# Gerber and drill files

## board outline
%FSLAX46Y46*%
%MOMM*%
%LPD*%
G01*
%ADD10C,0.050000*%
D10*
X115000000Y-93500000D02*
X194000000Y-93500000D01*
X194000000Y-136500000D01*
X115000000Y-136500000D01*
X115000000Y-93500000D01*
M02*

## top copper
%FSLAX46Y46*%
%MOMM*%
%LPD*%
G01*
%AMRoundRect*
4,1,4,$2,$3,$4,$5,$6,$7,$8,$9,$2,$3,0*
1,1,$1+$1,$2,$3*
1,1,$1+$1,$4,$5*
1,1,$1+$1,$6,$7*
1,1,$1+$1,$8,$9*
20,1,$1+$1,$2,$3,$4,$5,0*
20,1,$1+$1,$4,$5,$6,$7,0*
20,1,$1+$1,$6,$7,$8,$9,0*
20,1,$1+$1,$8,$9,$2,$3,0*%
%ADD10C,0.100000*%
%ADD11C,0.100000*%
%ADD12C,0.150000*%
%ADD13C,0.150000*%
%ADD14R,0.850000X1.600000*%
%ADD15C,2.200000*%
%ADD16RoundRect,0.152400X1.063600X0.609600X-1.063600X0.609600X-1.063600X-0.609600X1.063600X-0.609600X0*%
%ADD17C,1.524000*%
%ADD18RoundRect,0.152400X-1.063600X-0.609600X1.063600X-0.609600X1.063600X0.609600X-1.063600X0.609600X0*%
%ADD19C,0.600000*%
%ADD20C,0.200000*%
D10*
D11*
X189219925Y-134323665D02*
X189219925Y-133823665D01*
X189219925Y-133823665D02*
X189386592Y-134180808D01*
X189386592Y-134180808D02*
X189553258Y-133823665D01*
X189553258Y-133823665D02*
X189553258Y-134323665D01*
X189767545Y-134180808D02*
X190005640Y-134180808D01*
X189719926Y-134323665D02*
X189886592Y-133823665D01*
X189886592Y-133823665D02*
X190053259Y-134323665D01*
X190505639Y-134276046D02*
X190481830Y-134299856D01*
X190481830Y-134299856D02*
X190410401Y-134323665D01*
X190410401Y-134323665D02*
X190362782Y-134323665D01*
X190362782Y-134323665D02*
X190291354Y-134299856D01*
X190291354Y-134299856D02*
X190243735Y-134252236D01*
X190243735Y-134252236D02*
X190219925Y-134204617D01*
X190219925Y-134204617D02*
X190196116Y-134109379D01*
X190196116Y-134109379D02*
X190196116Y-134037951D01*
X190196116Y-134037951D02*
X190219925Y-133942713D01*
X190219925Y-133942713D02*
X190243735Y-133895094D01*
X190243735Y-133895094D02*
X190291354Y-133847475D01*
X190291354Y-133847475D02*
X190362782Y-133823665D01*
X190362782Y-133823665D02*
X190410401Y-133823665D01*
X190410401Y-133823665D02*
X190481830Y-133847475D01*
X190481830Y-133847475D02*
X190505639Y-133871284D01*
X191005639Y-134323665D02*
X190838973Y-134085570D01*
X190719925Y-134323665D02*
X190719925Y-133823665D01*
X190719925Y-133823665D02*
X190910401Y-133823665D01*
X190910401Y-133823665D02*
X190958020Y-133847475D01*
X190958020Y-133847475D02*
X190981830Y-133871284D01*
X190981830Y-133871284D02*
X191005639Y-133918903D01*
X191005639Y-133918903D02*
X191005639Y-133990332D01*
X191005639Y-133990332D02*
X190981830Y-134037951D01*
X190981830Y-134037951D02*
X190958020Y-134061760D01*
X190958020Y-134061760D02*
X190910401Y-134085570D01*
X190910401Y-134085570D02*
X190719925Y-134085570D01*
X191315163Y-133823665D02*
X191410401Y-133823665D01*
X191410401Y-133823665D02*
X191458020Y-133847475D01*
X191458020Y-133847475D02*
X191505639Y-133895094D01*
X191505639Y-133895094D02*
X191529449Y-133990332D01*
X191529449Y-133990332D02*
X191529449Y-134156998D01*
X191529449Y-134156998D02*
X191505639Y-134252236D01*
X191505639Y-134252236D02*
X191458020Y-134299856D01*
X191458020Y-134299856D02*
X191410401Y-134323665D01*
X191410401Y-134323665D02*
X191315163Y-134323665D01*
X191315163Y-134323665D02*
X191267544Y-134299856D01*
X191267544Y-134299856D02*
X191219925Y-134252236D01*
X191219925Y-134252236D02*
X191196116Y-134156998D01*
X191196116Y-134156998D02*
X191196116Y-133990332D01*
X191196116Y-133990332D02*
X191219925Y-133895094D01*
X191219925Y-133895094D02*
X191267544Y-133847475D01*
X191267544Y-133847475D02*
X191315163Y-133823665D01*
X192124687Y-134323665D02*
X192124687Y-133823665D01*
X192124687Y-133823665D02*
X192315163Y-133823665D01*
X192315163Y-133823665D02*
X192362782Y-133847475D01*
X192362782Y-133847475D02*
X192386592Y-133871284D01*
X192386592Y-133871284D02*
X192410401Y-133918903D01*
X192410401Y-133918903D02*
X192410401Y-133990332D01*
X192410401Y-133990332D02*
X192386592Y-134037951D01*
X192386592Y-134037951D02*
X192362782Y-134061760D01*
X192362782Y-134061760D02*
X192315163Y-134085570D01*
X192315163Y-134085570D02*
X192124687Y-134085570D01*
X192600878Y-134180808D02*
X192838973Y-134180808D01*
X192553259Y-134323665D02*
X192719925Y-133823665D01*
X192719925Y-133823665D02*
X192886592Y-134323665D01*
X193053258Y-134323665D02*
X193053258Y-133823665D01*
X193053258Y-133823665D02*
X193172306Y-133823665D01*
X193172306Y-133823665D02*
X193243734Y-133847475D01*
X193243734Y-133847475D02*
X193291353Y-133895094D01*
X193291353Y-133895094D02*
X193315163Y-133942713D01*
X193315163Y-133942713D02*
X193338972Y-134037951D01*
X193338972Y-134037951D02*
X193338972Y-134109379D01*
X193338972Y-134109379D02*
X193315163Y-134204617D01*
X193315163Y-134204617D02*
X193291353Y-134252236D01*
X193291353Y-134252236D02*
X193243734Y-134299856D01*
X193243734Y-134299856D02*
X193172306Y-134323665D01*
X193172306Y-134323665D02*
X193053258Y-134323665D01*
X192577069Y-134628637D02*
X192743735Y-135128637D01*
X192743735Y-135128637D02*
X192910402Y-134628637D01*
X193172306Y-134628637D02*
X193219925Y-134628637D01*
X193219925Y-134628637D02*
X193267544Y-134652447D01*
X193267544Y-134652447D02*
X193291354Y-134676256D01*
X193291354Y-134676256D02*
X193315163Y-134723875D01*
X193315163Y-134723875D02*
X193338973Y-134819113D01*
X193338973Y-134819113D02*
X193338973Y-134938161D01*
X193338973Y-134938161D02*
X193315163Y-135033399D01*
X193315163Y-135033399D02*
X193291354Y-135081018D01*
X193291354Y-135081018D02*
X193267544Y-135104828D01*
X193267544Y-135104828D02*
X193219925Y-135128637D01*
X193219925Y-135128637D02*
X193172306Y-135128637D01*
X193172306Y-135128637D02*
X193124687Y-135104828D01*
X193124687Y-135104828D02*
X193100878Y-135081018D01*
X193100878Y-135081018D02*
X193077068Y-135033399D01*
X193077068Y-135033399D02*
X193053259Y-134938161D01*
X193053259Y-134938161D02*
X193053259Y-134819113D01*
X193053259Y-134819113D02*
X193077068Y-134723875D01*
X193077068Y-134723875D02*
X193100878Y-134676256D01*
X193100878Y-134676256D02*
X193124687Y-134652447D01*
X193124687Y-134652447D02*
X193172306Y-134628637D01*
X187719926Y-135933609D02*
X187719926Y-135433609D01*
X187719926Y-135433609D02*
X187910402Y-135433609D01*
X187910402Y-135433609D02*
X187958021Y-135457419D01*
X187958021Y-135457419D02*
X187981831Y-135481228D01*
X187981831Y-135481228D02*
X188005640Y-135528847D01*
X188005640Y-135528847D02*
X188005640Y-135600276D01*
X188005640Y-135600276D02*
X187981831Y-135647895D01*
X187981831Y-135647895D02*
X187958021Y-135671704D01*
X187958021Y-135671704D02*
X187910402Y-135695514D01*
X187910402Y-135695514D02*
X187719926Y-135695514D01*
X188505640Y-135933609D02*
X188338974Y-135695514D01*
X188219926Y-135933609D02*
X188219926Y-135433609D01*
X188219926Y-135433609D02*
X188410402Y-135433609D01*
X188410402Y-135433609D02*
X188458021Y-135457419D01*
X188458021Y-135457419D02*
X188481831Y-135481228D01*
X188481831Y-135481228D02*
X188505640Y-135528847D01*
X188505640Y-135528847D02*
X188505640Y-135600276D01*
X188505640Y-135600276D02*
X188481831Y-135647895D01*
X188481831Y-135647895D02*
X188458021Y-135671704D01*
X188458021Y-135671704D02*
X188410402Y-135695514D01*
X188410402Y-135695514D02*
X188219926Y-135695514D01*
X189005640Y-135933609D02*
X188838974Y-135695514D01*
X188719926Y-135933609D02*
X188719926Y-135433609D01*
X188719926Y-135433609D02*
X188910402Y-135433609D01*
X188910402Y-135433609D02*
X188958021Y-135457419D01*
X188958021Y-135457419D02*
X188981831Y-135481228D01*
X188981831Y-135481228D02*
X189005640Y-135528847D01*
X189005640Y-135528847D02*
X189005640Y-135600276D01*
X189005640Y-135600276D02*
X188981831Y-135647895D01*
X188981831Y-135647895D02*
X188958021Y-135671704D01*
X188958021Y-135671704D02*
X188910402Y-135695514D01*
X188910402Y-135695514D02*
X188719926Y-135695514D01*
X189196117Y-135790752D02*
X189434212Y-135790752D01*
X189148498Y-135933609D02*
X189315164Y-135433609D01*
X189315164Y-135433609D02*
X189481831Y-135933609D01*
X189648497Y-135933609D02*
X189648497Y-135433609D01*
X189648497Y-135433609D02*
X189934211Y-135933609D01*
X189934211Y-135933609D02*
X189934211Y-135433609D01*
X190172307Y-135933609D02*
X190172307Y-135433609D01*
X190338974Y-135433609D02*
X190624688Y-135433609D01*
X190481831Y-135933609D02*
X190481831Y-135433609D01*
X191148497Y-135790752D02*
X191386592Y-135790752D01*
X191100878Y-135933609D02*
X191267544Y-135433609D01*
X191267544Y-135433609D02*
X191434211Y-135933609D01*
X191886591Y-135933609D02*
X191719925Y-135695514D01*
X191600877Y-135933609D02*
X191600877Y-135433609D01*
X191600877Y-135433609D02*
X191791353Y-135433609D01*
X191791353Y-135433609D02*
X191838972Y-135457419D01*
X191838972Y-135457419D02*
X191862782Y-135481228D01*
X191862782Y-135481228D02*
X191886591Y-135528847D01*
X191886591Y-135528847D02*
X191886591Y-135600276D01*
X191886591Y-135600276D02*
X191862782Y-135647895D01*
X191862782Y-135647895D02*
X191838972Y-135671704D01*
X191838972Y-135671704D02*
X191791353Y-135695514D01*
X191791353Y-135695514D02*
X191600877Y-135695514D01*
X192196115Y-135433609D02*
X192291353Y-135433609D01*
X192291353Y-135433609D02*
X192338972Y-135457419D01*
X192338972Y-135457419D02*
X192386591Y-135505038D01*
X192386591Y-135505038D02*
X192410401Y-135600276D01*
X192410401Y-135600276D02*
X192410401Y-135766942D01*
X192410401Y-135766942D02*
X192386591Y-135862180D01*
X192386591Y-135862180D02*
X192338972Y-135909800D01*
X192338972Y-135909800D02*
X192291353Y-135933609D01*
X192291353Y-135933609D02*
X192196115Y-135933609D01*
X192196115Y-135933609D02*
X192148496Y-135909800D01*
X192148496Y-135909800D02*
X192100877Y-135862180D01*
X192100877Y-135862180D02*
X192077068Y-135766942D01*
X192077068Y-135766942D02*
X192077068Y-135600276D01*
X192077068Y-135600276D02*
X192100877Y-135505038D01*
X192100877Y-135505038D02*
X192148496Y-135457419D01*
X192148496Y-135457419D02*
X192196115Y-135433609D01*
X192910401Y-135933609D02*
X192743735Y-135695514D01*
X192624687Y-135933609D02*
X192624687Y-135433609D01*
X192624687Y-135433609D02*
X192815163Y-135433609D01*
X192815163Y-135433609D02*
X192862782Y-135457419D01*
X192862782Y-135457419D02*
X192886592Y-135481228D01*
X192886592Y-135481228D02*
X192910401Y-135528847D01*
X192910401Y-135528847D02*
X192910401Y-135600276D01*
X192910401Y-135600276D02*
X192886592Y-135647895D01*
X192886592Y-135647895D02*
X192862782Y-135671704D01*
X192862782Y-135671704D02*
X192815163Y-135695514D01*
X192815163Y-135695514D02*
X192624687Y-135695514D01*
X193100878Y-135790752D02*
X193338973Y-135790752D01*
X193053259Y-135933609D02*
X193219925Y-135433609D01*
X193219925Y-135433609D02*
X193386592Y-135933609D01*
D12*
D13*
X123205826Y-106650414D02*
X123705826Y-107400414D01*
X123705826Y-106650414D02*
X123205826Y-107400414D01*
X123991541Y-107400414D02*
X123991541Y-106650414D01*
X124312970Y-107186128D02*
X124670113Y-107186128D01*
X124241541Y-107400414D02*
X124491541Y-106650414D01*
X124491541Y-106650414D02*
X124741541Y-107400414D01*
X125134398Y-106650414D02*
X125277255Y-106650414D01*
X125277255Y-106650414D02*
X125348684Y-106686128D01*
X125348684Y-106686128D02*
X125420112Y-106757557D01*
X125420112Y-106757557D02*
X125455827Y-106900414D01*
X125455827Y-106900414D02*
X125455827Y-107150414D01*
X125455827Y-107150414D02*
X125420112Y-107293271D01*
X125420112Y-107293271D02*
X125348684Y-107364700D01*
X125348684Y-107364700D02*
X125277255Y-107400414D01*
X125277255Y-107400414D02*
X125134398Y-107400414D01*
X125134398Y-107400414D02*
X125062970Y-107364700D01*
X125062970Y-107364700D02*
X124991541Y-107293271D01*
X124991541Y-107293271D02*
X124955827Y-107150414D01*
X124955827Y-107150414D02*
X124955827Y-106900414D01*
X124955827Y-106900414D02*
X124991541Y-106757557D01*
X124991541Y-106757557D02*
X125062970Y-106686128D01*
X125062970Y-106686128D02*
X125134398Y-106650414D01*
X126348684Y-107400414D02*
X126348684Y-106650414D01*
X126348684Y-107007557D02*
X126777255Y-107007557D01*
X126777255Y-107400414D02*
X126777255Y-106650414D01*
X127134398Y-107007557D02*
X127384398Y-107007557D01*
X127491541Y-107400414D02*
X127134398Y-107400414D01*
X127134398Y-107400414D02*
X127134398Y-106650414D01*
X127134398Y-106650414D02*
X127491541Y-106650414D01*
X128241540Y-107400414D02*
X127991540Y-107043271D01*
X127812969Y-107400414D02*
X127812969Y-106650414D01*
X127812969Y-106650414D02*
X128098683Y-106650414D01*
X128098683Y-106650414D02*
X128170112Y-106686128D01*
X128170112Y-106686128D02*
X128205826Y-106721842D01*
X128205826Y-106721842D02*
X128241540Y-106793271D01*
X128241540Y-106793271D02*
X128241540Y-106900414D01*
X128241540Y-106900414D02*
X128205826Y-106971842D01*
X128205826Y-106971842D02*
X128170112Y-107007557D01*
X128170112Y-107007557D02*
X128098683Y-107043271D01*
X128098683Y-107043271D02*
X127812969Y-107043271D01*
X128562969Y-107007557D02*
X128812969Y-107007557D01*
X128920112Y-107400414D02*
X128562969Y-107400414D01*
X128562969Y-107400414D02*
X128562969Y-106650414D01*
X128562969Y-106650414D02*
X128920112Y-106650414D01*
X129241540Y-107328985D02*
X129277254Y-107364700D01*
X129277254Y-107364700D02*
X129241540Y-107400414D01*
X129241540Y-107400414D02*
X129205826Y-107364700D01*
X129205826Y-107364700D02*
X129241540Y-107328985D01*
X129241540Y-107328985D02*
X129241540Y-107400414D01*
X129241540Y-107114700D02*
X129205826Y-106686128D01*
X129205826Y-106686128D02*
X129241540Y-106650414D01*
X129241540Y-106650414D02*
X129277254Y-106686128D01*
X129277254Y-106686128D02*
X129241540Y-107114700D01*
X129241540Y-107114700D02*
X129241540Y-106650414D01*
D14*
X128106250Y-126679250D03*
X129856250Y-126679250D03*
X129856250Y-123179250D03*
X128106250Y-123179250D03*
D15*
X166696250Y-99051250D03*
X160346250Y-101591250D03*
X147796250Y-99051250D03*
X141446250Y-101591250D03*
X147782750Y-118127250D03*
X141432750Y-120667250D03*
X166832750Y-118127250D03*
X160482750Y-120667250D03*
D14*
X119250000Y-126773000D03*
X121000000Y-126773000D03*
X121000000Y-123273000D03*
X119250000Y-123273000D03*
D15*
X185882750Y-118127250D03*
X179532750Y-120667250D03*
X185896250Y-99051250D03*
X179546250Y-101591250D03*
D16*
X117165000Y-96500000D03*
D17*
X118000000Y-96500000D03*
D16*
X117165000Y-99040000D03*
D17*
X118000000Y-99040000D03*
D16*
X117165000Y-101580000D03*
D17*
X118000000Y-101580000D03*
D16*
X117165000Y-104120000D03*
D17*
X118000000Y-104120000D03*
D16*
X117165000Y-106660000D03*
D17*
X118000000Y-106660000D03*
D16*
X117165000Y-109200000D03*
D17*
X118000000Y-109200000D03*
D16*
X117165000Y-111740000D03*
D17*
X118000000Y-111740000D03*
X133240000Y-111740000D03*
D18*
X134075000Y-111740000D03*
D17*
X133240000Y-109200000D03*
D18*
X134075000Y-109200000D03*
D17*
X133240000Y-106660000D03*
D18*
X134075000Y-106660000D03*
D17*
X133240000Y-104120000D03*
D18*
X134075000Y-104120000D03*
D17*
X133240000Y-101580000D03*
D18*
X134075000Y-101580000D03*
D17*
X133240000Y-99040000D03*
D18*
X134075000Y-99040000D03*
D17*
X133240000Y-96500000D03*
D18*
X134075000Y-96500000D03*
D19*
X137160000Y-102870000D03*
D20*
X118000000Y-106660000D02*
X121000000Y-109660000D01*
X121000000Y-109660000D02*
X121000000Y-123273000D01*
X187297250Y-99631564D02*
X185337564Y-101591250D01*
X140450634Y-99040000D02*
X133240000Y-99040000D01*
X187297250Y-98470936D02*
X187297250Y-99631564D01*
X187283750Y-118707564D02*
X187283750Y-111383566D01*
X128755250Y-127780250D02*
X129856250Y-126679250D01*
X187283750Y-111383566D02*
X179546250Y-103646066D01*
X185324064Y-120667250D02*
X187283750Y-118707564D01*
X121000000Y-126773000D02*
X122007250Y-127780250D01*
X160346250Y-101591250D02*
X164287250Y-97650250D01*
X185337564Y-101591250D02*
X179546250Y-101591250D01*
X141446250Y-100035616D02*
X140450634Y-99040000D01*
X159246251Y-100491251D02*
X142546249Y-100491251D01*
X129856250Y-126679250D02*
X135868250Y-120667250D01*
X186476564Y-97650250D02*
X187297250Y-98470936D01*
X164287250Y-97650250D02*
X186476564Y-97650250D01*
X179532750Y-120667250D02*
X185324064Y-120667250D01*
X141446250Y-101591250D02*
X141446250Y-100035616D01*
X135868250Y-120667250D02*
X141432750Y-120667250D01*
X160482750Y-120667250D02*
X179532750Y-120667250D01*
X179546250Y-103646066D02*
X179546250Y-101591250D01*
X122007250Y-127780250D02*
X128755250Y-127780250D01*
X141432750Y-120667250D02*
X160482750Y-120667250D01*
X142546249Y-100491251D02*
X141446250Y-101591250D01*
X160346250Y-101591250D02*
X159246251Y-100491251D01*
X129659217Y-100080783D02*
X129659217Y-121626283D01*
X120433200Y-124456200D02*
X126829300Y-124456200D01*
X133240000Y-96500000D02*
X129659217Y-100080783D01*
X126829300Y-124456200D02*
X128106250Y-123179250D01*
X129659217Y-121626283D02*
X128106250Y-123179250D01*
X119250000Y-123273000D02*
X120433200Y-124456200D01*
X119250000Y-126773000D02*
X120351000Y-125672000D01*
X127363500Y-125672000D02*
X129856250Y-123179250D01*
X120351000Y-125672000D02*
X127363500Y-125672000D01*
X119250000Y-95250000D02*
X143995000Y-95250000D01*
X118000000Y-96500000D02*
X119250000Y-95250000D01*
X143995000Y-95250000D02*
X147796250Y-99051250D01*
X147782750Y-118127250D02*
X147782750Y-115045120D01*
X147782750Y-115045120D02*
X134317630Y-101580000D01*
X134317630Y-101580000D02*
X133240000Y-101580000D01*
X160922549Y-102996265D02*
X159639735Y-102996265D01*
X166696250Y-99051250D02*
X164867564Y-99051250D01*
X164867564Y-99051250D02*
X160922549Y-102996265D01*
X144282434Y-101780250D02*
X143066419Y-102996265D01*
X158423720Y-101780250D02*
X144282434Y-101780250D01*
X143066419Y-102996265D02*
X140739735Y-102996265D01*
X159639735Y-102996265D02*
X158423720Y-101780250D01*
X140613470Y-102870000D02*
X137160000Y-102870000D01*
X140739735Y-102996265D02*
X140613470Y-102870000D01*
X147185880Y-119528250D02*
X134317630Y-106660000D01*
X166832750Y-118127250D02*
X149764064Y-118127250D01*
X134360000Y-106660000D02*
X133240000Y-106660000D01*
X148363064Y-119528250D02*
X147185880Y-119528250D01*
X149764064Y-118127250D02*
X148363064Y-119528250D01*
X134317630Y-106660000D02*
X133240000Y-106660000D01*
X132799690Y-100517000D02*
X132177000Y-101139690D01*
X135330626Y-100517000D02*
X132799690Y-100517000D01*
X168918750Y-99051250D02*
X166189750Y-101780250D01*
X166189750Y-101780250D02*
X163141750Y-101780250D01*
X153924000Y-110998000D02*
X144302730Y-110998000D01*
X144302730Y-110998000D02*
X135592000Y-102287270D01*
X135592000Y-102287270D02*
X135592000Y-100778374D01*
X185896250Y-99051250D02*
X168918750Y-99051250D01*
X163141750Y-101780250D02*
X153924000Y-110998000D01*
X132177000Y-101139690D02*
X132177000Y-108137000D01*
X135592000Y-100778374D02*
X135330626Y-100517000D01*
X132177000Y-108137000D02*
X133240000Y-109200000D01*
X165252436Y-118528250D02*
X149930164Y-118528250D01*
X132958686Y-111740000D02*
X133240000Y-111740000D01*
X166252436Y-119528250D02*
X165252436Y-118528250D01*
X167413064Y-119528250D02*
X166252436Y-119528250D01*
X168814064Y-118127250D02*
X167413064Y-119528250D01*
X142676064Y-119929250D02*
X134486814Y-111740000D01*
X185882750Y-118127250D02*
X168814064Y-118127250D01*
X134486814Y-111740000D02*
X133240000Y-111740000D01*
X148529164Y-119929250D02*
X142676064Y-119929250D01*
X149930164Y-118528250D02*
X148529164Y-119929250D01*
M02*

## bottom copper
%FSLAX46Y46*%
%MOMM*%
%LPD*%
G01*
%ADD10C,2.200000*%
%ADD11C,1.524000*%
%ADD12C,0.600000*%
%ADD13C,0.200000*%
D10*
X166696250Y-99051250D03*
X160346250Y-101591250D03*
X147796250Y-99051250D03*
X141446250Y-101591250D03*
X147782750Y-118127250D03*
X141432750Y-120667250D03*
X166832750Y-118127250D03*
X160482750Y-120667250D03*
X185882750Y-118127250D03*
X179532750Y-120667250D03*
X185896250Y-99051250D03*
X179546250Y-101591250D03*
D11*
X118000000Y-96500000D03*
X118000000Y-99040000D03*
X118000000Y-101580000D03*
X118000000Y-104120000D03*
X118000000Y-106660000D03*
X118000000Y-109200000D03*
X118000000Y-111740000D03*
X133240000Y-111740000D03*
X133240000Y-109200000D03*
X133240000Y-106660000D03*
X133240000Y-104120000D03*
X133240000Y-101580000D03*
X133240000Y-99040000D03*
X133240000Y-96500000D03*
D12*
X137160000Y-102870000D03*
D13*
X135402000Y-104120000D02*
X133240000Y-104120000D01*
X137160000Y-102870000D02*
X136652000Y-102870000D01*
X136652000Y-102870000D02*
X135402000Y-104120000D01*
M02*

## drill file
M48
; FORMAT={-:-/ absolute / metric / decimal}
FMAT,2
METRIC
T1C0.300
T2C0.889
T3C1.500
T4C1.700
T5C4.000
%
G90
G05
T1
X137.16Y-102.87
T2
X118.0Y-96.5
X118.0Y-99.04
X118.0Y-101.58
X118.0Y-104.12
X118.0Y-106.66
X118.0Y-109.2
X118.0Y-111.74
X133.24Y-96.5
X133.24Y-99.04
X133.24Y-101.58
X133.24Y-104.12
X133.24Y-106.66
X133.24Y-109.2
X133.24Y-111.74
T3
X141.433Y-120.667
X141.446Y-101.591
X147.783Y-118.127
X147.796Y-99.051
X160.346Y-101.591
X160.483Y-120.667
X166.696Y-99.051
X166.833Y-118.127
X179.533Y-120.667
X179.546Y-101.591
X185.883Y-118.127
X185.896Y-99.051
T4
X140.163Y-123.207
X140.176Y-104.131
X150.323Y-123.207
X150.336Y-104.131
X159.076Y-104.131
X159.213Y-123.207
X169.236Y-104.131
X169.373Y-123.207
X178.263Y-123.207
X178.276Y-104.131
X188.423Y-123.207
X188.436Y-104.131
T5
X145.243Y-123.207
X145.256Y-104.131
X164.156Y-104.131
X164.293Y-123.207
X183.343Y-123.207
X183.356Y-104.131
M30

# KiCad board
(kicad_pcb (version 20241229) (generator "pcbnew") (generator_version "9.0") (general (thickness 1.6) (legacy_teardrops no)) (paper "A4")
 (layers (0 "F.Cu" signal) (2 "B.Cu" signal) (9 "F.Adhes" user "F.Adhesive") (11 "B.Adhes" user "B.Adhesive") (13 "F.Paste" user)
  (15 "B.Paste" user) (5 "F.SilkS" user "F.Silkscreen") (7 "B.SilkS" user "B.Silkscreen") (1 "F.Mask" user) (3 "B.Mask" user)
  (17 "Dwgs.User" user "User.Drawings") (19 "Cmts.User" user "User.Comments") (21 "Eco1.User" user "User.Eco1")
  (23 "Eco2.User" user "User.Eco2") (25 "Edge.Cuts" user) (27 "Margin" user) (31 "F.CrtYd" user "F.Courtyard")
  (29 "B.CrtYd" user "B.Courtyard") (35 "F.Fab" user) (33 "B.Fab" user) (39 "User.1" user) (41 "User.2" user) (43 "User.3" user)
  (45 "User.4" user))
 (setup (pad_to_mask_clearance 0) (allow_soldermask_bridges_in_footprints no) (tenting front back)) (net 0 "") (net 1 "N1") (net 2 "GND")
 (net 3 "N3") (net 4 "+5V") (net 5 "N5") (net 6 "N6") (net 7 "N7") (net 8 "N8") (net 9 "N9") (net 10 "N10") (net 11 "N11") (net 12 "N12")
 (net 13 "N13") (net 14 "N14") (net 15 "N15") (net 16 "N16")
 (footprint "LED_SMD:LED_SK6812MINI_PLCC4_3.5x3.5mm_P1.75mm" (layer "F.Cu") (at 128.98125 124.92925 90)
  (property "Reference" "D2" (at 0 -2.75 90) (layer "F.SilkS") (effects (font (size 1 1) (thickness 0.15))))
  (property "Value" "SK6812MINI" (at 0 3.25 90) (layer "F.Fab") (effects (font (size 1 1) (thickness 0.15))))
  (pad "1" smd rect (at -1.75 -0.875 90) (size 1.6 0.85) (layers "F.Cu" "F.Mask" "F.Paste") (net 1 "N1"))
  (pad "2" smd rect (at -1.75 0.875 90) (size 1.6 0.85) (layers "F.Cu" "F.Mask" "F.Paste") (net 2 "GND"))
  (pad "3" smd rect (at 1.75 0.875 90) (size 1.6 0.85) (layers "F.Cu" "F.Mask" "F.Paste") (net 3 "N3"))
  (pad "4" smd rect (at 1.75 -0.875 90) (size 1.6 0.85) (layers "F.Cu" "F.Mask" "F.Paste") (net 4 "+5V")))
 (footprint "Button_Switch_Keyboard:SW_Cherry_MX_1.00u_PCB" (layer "F.Cu") (at 166.69625 99.05125)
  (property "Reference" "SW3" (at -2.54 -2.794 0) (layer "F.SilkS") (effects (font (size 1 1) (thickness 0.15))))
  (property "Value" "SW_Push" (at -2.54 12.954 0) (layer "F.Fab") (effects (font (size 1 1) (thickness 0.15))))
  (pad "" np_thru_hole circle (at -7.62 5.08) (size 1.7 1.7) (drill 1.7) (layers "*.Cu" "*.Mask"))
  (pad "" np_thru_hole circle (at -2.54 5.08) (size 4 4) (drill 4) (layers "*.Cu" "*.Mask"))
  (pad "" np_thru_hole circle (at 2.54 5.08) (size 1.7 1.7) (drill 1.7) (layers "*.Cu" "*.Mask"))
  (pad "1" thru_hole circle (at 0 0) (size 2.2 2.2) (drill 1.5) (layers "*.Cu" "*.Mask") (remove_unused_layers no) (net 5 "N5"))
  (pad "2" thru_hole circle (at -6.35 2.54) (size 2.2 2.2) (drill 1.5) (layers "*.Cu" "*.Mask") (remove_unused_layers no) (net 2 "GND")))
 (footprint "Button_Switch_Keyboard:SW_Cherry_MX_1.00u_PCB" (layer "F.Cu") (at 147.79625 99.05125)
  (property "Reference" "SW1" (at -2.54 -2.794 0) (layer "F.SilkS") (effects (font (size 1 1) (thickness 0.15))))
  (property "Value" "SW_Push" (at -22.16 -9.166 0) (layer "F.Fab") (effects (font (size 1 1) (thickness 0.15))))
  (pad "" np_thru_hole circle (at -7.62 5.08) (size 1.7 1.7) (drill 1.7) (layers "*.Cu" "*.Mask"))
  (pad "" np_thru_hole circle (at -2.54 5.08) (size 4 4) (drill 4) (layers "*.Cu" "*.Mask"))
  (pad "" np_thru_hole circle (at 2.54 5.08) (size 1.7 1.7) (drill 1.7) (layers "*.Cu" "*.Mask"))
  (pad "1" thru_hole circle (at 0 0) (size 2.2 2.2) (drill 1.5) (layers "*.Cu" "*.Mask") (remove_unused_layers no) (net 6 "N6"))
  (pad "2" thru_hole circle (at -6.35 2.54) (size 2.2 2.2) (drill 1.5) (layers "*.Cu" "*.Mask") (remove_unused_layers no) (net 2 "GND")))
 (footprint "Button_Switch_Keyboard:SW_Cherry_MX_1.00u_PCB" (layer "F.Cu") (at 147.78275 118.12725)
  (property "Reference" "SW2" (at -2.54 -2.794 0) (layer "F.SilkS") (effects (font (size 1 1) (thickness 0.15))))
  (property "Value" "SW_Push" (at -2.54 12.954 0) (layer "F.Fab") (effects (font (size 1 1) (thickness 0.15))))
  (pad "" np_thru_hole circle (at -7.62 5.08) (size 1.7 1.7) (drill 1.7) (layers "*.Cu" "*.Mask"))
  (pad "" np_thru_hole circle (at -2.54 5.08) (size 4 4) (drill 4) (layers "*.Cu" "*.Mask"))
  (pad "" np_thru_hole circle (at 2.54 5.08) (size 1.7 1.7) (drill 1.7) (layers "*.Cu" "*.Mask"))
  (pad "1" thru_hole circle (at 0 0) (size 2.2 2.2) (drill 1.5) (layers "*.Cu" "*.Mask") (remove_unused_layers no) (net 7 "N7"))
  (pad "2" thru_hole circle (at -6.35 2.54) (size 2.2 2.2) (drill 1.5) (layers "*.Cu" "*.Mask") (remove_unused_layers no) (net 2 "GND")))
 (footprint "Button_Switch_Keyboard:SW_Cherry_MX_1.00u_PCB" (layer "F.Cu") (at 166.83275 118.12725)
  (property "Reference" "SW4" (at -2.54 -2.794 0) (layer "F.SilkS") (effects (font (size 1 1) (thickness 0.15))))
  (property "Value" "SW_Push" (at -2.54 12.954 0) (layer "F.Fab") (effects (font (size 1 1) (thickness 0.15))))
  (pad "" np_thru_hole circle (at -7.62 5.08) (size 1.7 1.7) (drill 1.7) (layers "*.Cu" "*.Mask"))
  (pad "" np_thru_hole circle (at -2.54 5.08) (size 4 4) (drill 4) (layers "*.Cu" "*.Mask"))
  (pad "" np_thru_hole circle (at 2.54 5.08) (size 1.7 1.7) (drill 1.7) (layers "*.Cu" "*.Mask"))
  (pad "1" thru_hole circle (at 0 0) (size 2.2 2.2) (drill 1.5) (layers "*.Cu" "*.Mask") (remove_unused_layers no) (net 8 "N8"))
  (pad "2" thru_hole circle (at -6.35 2.54) (size 2.2 2.2) (drill 1.5) (layers "*.Cu" "*.Mask") (remove_unused_layers no) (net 2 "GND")))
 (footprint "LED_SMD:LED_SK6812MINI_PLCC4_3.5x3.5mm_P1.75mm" (layer "F.Cu") (at 120.125 125.023 90)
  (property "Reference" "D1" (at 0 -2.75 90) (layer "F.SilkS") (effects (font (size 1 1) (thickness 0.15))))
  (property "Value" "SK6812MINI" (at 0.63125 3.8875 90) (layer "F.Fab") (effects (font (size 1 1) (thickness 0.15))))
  (pad "1" smd rect (at -1.75 -0.875 90) (size 1.6 0.85) (layers "F.Cu" "F.Mask" "F.Paste") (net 3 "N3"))
  (pad "2" smd rect (at -1.75 0.875 90) (size 1.6 0.85) (layers "F.Cu" "F.Mask" "F.Paste") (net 2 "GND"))
  (pad "3" smd rect (at 1.75 0.875 90) (size 1.6 0.85) (layers "F.Cu" "F.Mask" "F.Paste") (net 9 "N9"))
  (pad "4" smd rect (at 1.75 -0.875 90) (size 1.6 0.85) (layers "F.Cu" "F.Mask" "F.Paste") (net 4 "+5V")))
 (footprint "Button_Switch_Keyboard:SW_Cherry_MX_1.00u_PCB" (layer "F.Cu") (at 185.88275 118.12725)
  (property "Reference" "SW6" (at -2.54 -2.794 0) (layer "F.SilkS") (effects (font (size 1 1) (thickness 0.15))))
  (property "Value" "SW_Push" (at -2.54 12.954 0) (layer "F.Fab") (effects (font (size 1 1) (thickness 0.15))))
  (pad "" np_thru_hole circle (at -7.62 5.08) (size 1.7 1.7) (drill 1.7) (layers "*.Cu" "*.Mask"))
  (pad "" np_thru_hole circle (at -2.54 5.08) (size 4 4) (drill 4) (layers "*.Cu" "*.Mask"))
  (pad "" np_thru_hole circle (at 2.54 5.08) (size 1.7 1.7) (drill 1.7) (layers "*.Cu" "*.Mask"))
  (pad "1" thru_hole circle (at 0 0) (size 2.2 2.2) (drill 1.5) (layers "*.Cu" "*.Mask") (remove_unused_layers no) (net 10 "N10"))
  (pad "2" thru_hole circle (at -6.35 2.54) (size 2.2 2.2) (drill 1.5) (layers "*.Cu" "*.Mask") (remove_unused_layers no) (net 2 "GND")))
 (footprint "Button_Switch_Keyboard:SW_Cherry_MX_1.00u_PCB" (layer "F.Cu") (at 185.89625 99.05125)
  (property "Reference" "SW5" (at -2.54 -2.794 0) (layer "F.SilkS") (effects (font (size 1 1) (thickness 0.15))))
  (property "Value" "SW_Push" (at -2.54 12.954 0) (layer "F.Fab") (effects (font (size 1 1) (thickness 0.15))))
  (pad "" np_thru_hole circle (at -7.62 5.08) (size 1.7 1.7) (drill 1.7) (layers "*.Cu" "*.Mask"))
  (pad "" np_thru_hole circle (at -2.54 5.08) (size 4 4) (drill 4) (layers "*.Cu" "*.Mask"))
  (pad "" np_thru_hole circle (at 2.54 5.08) (size 1.7 1.7) (drill 1.7) (layers "*.Cu" "*.Mask"))
  (pad "1" thru_hole circle (at 0 0) (size 2.2 2.2) (drill 1.5) (layers "*.Cu" "*.Mask") (remove_unused_layers no) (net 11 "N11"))
  (pad "2" thru_hole circle (at -6.35 2.54) (size 2.2 2.2) (drill 1.5) (layers "*.Cu" "*.Mask") (remove_unused_layers no) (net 2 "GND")))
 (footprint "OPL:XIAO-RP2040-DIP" (layer "F.Cu") (at 125.62 104.12)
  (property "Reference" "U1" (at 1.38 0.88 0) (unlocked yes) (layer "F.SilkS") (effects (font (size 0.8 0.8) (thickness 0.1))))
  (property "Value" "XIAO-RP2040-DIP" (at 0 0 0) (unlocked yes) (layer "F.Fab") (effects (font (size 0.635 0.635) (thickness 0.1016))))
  (pad "1" smd roundrect (at -8.455 -7.62 180) (size 2.432 1.524) (layers "F.Cu" "F.Mask") (roundrect_rratio 0.1) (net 6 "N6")
   (thermal_bridge_angle 45))
  (pad "1" thru_hole circle (at -7.62 -7.62 180) (size 1.524 1.524) (drill 0.889) (layers "*.Cu" "*.Mask") (remove_unused_layers no)
   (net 6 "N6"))
  (pad "2" smd roundrect (at -8.455 -5.08 180) (size 2.432 1.524) (layers "F.Cu" "F.Mask") (roundrect_rratio 0.1) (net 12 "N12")
   (thermal_bridge_angle 45))
  (pad "2" thru_hole circle (at -7.62 -5.08 180) (size 1.524 1.524) (drill 0.889) (layers "*.Cu" "*.Mask") (remove_unused_layers no)
   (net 12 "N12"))
  (pad "3" smd roundrect (at -8.455 -2.54 180) (size 2.432 1.524) (layers "F.Cu" "F.Mask") (roundrect_rratio 0.1) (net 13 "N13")
   (thermal_bridge_angle 45))
  (pad "3" thru_hole circle (at -7.62 -2.54 180) (size 1.524 1.524) (drill 0.889) (layers "*.Cu" "*.Mask") (remove_unused_layers no)
   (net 13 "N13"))
  (pad "4" smd roundrect (at -8.455 0 180) (size 2.432 1.524) (layers "F.Cu" "F.Mask") (roundrect_rratio 0.1) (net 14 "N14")
   (thermal_bridge_angle 45))
  (pad "4" thru_hole circle (at -7.62 0 180) (size 1.524 1.524) (drill 0.889) (layers "*.Cu" "*.Mask") (remove_unused_layers no)
   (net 14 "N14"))
  (pad "5" smd roundrect (at -8.455 2.54 180) (size 2.432 1.524) (layers "F.Cu" "F.Mask") (roundrect_rratio 0.1) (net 9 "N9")
   (thermal_bridge_angle 45))
  (pad "5" thru_hole circle (at -7.62 2.54 180) (size 1.524 1.524) (drill 0.889) (layers "*.Cu" "*.Mask") (remove_unused_layers no)
   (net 9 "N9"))
  (pad "6" smd roundrect (at -8.455 5.08 180) (size 2.432 1.524) (layers "F.Cu" "F.Mask") (roundrect_rratio 0.1) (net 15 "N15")
   (thermal_bridge_angle 45))
  (pad "6" thru_hole circle (at -7.62 5.08 180) (size 1.524 1.524) (drill 0.889) (layers "*.Cu" "*.Mask") (remove_unused_layers no)
   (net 15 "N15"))
  (pad "7" smd roundrect (at -8.455 7.62 180) (size 2.432 1.524) (layers "F.Cu" "F.Mask") (roundrect_rratio 0.1) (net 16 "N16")
   (thermal_bridge_angle 45))
  (pad "7" thru_hole circle (at -7.62 7.62 180) (size 1.524 1.524) (drill 0.889) (layers "*.Cu" "*.Mask") (remove_unused_layers no)
   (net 16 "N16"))
  (pad "8" thru_hole circle (at 7.62 7.62) (size 1.524 1.524) (drill 0.889) (layers "*.Cu" "*.Mask") (remove_unused_layers no)
   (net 10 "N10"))
  (pad "8" smd roundrect (at 8.455 7.62) (size 2.432 1.524) (layers "F.Cu" "F.Mask") (roundrect_rratio 0.1) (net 10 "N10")
   (thermal_bridge_angle 45))
  (pad "9" thru_hole circle (at 7.62 5.08) (size 1.524 1.524) (drill 0.889) (layers "*.Cu" "*.Mask") (remove_unused_layers no)
   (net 11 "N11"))
  (pad "9" smd roundrect (at 8.455 5.08) (size 2.432 1.524) (layers "F.Cu" "F.Mask") (roundrect_rratio 0.1) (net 11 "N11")
   (thermal_bridge_angle 45))
  (pad "10" thru_hole circle (at 7.62 2.54) (size 1.524 1.524) (drill 0.889) (layers "*.Cu" "*.Mask") (remove_unused_layers no) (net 8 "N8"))
  (pad "10" smd roundrect (at 8.455 2.54) (size 2.432 1.524) (layers "F.Cu" "F.Mask") (roundrect_rratio 0.1) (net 8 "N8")
   (thermal_bridge_angle 45))
  (pad "11" thru_hole circle (at 7.62 0) (size 1.524 1.524) (drill 0.889) (layers "*.Cu" "*.Mask") (remove_unused_layers no) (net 5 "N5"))
  (pad "11" smd roundrect (at 8.455 0) (size 2.432 1.524) (layers "F.Cu" "F.Mask") (roundrect_rratio 0.1) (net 5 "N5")
   (thermal_bridge_angle 45))
  (pad "12" thru_hole circle (at 7.62 -2.54) (size 1.524 1.524) (drill 0.889) (layers "*.Cu" "*.Mask") (remove_unused_layers no)
   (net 7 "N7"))
  (pad "12" smd roundrect (at 8.455 -2.54) (size 2.432 1.524) (layers "F.Cu" "F.Mask") (roundrect_rratio 0.1) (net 7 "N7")
   (thermal_bridge_angle 45))
  (pad "13" thru_hole circle (at 7.62 -5.08) (size 1.524 1.524) (drill 0.889) (layers "*.Cu" "*.Mask") (remove_unused_layers no)
   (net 2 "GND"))
  (pad "13" smd roundrect (at 8.455 -5.08) (size 2.432 1.524) (layers "F.Cu" "F.Mask") (roundrect_rratio 0.1) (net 2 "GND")
   (thermal_bridge_angle 45))
  (pad "14" thru_hole circle (at 7.62 -7.62) (size 1.524 1.524) (drill 0.889) (layers "*.Cu" "*.Mask") (remove_unused_layers no)
   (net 4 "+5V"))
  (pad "14" smd roundrect (at 8.455 -7.62) (size 2.432 1.524) (layers "F.Cu" "F.Mask") (roundrect_rratio 0.1) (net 4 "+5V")
   (thermal_bridge_angle 45)))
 (gr_rect (start 115 93.5) (end 194 136.5) (stroke (width 0.05) (type default)) (fill no) (layer "Edge.Cuts"))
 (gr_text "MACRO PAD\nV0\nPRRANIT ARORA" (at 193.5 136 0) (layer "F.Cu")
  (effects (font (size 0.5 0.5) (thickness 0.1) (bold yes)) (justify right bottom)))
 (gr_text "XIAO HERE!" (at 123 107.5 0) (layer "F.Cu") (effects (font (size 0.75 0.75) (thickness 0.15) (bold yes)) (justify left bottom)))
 (segment (start 118 106.66) (end 121 109.66) (width 0.2) (layer "F.Cu") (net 9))
 (segment (start 121 109.66) (end 121 123.273) (width 0.2) (layer "F.Cu") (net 9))
 (segment (start 187.29725 99.631564) (end 185.337564 101.59125) (width 0.2) (layer "F.Cu") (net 2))
 (segment (start 140.450634 99.04) (end 133.24 99.04) (width 0.2) (layer "F.Cu") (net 2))
 (segment (start 187.29725 98.470936) (end 187.29725 99.631564) (width 0.2) (layer "F.Cu") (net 2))
 (segment (start 187.28375 118.707564) (end 187.28375 111.383566) (width 0.2) (layer "F.Cu") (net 2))
 (segment (start 128.75525 127.78025) (end 129.85625 126.67925) (width 0.2) (layer "F.Cu") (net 2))
 (segment (start 187.28375 111.383566) (end 179.54625 103.646066) (width 0.2) (layer "F.Cu") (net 2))
 (segment (start 185.324064 120.66725) (end 187.28375 118.707564) (width 0.2) (layer "F.Cu") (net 2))
 (segment (start 121 126.773) (end 122.00725 127.78025) (width 0.2) (layer "F.Cu") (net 2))
 (segment (start 160.34625 101.59125) (end 164.28725 97.65025) (width 0.2) (layer "F.Cu") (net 2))
 (segment (start 185.337564 101.59125) (end 179.54625 101.59125) (width 0.2) (layer "F.Cu") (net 2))
 (segment (start 141.44625 100.035616) (end 140.450634 99.04) (width 0.2) (layer "F.Cu") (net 2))
 (segment (start 159.246251 100.491251) (end 142.546249 100.491251) (width 0.2) (layer "F.Cu") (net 2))
 (segment (start 129.85625 126.67925) (end 135.86825 120.66725) (width 0.2) (layer "F.Cu") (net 2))
 (segment (start 186.476564 97.65025) (end 187.29725 98.470936) (width 0.2) (layer "F.Cu") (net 2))
 (segment (start 164.28725 97.65025) (end 186.476564 97.65025) (width 0.2) (layer "F.Cu") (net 2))
 (segment (start 179.53275 120.66725) (end 185.324064 120.66725) (width 0.2) (layer "F.Cu") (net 2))
 (segment (start 141.44625 101.59125) (end 141.44625 100.035616) (width 0.2) (layer "F.Cu") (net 2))
 (segment (start 135.86825 120.66725) (end 141.43275 120.66725) (width 0.2) (layer "F.Cu") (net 2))
 (segment (start 160.48275 120.66725) (end 179.53275 120.66725) (width 0.2) (layer "F.Cu") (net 2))
 (segment (start 179.54625 103.646066) (end 179.54625 101.59125) (width 0.2) (layer "F.Cu") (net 2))
 (segment (start 122.00725 127.78025) (end 128.75525 127.78025) (width 0.2) (layer "F.Cu") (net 2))
 (segment (start 141.43275 120.66725) (end 160.48275 120.66725) (width 0.2) (layer "F.Cu") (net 2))
 (segment (start 142.546249 100.491251) (end 141.44625 101.59125) (width 0.2) (layer "F.Cu") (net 2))
 (segment (start 160.34625 101.59125) (end 159.246251 100.491251) (width 0.2) (layer "F.Cu") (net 2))
 (segment (start 129.659217 100.080783) (end 129.659217 121.626283) (width 0.2) (layer "F.Cu") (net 4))
 (segment (start 120.4332 124.4562) (end 126.8293 124.4562) (width 0.2) (layer "F.Cu") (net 4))
 (segment (start 133.24 96.5) (end 129.659217 100.080783) (width 0.2) (layer "F.Cu") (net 4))
 (segment (start 126.8293 124.4562) (end 128.10625 123.17925) (width 0.2) (layer "F.Cu") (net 4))
 (segment (start 129.659217 121.626283) (end 128.10625 123.17925) (width 0.2) (layer "F.Cu") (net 4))
 (segment (start 119.25 123.273) (end 120.4332 124.4562) (width 0.2) (layer "F.Cu") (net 4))
 (segment (start 119.25 126.773) (end 120.351 125.672) (width 0.2) (layer "F.Cu") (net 3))
 (segment (start 127.3635 125.672) (end 129.85625 123.17925) (width 0.2) (layer "F.Cu") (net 3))
 (segment (start 120.351 125.672) (end 127.3635 125.672) (width 0.2) (layer "F.Cu") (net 3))
 (segment (start 119.25 95.25) (end 143.995 95.25) (width 0.2) (layer "F.Cu") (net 6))
 (segment (start 118 96.5) (end 119.25 95.25) (width 0.2) (layer "F.Cu") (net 6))
 (segment (start 143.995 95.25) (end 147.79625 99.05125) (width 0.2) (layer "F.Cu") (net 6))
 (segment (start 147.78275 118.12725) (end 147.78275 115.04512) (width 0.2) (layer "F.Cu") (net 7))
 (segment (start 147.78275 115.04512) (end 134.31763 101.58) (width 0.2) (layer "F.Cu") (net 7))
 (segment (start 134.31763 101.58) (end 133.24 101.58) (width 0.2) (layer "F.Cu") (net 7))
 (segment (start 160.922549 102.996265) (end 159.639735 102.996265) (width 0.2) (layer "F.Cu") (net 5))
 (segment (start 166.69625 99.05125) (end 164.867564 99.05125) (width 0.2) (layer "F.Cu") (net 5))
 (segment (start 164.867564 99.05125) (end 160.922549 102.996265) (width 0.2) (layer "F.Cu") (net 5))
 (segment (start 144.282434 101.78025) (end 143.066419 102.996265) (width 0.2) (layer "F.Cu") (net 5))
 (segment (start 158.42372 101.78025) (end 144.282434 101.78025) (width 0.2) (layer "F.Cu") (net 5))
 (segment (start 143.066419 102.996265) (end 140.739735 102.996265) (width 0.2) (layer "F.Cu") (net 5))
 (segment (start 159.639735 102.996265) (end 158.42372 101.78025) (width 0.2) (layer "F.Cu") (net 5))
 (segment (start 140.61347 102.87) (end 137.16 102.87) (width 0.2) (layer "F.Cu") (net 5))
 (segment (start 140.739735 102.996265) (end 140.61347 102.87) (width 0.2) (layer "F.Cu") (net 5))
 (via (at 137.16 102.87) (size 0.6) (drill 0.3) (layers "F.Cu" "B.Cu") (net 5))
 (segment (start 135.402 104.12) (end 133.24 104.12) (width 0.2) (layer "B.Cu") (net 5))
 (segment (start 137.16 102.87) (end 136.652 102.87) (width 0.2) (layer "B.Cu") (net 5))
 (segment (start 136.652 102.87) (end 135.402 104.12) (width 0.2) (layer "B.Cu") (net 5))
 (segment (start 147.18588 119.52825) (end 134.31763 106.66) (width 0.2) (layer "F.Cu") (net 8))
 (segment (start 166.83275 118.12725) (end 149.764064 118.12725) (width 0.2) (layer "F.Cu") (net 8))
 (segment (start 134.36 106.66) (end 133.24 106.66) (width 0.2) (layer "F.Cu") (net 8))
 (segment (start 148.363064 119.52825) (end 147.18588 119.52825) (width 0.2) (layer "F.Cu") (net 8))
 (segment (start 149.764064 118.12725) (end 148.363064 119.52825) (width 0.2) (layer "F.Cu") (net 8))
 (segment (start 134.31763 106.66) (end 133.24 106.66) (width 0.2) (layer "F.Cu") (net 8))
 (segment (start 132.79969 100.517) (end 132.177 101.13969) (width 0.2) (layer "F.Cu") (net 11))
 (segment (start 135.330626 100.517) (end 132.79969 100.517) (width 0.2) (layer "F.Cu") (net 11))
 (segment (start 168.91875 99.05125) (end 166.18975 101.78025) (width 0.2) (layer "F.Cu") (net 11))
 (segment (start 166.18975 101.78025) (end 163.14175 101.78025) (width 0.2) (layer "F.Cu") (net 11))
 (segment (start 153.924 110.998) (end 144.30273 110.998) (width 0.2) (layer "F.Cu") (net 11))
 (segment (start 144.30273 110.998) (end 135.592 102.28727) (width 0.2) (layer "F.Cu") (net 11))
 (segment (start 135.592 102.28727) (end 135.592 100.778374) (width 0.2) (layer "F.Cu") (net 11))
 (segment (start 185.89625 99.05125) (end 168.91875 99.05125) (width 0.2) (layer "F.Cu") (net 11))
 (segment (start 163.14175 101.78025) (end 153.924 110.998) (width 0.2) (layer "F.Cu") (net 11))
 (segment (start 132.177 101.13969) (end 132.177 108.137) (width 0.2) (layer "F.Cu") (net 11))
 (segment (start 135.592 100.778374) (end 135.330626 100.517) (width 0.2) (layer "F.Cu") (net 11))
 (segment (start 132.177 108.137) (end 133.24 109.2) (width 0.2) (layer "F.Cu") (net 11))
 (segment (start 165.252436 118.52825) (end 149.930164 118.52825) (width 0.2) (layer "F.Cu") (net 10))
 (segment (start 132.958686 111.74) (end 133.24 111.74) (width 0.2) (layer "F.Cu") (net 10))
 (segment (start 166.252436 119.52825) (end 165.252436 118.52825) (width 0.2) (layer "F.Cu") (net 10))
 (segment (start 167.413064 119.52825) (end 166.252436 119.52825) (width 0.2) (layer "F.Cu") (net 10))
 (segment (start 168.814064 118.12725) (end 167.413064 119.52825) (width 0.2) (layer "F.Cu") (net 10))
 (segment (start 142.676064 119.92925) (end 134.486814 111.74) (width 0.2) (layer "F.Cu") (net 10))
 (segment (start 185.88275 118.12725) (end 168.814064 118.12725) (width 0.2) (layer "F.Cu") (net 10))
 (segment (start 134.486814 111.74) (end 133.24 111.74) (width 0.2) (layer "F.Cu") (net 10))
 (segment (start 148.529164 119.92925) (end 142.676064 119.92925) (width 0.2) (layer "F.Cu") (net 10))
 (segment (start 149.930164 118.52825) (end 148.529164 119.92925) (width 0.2) (layer "F.Cu") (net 10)))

